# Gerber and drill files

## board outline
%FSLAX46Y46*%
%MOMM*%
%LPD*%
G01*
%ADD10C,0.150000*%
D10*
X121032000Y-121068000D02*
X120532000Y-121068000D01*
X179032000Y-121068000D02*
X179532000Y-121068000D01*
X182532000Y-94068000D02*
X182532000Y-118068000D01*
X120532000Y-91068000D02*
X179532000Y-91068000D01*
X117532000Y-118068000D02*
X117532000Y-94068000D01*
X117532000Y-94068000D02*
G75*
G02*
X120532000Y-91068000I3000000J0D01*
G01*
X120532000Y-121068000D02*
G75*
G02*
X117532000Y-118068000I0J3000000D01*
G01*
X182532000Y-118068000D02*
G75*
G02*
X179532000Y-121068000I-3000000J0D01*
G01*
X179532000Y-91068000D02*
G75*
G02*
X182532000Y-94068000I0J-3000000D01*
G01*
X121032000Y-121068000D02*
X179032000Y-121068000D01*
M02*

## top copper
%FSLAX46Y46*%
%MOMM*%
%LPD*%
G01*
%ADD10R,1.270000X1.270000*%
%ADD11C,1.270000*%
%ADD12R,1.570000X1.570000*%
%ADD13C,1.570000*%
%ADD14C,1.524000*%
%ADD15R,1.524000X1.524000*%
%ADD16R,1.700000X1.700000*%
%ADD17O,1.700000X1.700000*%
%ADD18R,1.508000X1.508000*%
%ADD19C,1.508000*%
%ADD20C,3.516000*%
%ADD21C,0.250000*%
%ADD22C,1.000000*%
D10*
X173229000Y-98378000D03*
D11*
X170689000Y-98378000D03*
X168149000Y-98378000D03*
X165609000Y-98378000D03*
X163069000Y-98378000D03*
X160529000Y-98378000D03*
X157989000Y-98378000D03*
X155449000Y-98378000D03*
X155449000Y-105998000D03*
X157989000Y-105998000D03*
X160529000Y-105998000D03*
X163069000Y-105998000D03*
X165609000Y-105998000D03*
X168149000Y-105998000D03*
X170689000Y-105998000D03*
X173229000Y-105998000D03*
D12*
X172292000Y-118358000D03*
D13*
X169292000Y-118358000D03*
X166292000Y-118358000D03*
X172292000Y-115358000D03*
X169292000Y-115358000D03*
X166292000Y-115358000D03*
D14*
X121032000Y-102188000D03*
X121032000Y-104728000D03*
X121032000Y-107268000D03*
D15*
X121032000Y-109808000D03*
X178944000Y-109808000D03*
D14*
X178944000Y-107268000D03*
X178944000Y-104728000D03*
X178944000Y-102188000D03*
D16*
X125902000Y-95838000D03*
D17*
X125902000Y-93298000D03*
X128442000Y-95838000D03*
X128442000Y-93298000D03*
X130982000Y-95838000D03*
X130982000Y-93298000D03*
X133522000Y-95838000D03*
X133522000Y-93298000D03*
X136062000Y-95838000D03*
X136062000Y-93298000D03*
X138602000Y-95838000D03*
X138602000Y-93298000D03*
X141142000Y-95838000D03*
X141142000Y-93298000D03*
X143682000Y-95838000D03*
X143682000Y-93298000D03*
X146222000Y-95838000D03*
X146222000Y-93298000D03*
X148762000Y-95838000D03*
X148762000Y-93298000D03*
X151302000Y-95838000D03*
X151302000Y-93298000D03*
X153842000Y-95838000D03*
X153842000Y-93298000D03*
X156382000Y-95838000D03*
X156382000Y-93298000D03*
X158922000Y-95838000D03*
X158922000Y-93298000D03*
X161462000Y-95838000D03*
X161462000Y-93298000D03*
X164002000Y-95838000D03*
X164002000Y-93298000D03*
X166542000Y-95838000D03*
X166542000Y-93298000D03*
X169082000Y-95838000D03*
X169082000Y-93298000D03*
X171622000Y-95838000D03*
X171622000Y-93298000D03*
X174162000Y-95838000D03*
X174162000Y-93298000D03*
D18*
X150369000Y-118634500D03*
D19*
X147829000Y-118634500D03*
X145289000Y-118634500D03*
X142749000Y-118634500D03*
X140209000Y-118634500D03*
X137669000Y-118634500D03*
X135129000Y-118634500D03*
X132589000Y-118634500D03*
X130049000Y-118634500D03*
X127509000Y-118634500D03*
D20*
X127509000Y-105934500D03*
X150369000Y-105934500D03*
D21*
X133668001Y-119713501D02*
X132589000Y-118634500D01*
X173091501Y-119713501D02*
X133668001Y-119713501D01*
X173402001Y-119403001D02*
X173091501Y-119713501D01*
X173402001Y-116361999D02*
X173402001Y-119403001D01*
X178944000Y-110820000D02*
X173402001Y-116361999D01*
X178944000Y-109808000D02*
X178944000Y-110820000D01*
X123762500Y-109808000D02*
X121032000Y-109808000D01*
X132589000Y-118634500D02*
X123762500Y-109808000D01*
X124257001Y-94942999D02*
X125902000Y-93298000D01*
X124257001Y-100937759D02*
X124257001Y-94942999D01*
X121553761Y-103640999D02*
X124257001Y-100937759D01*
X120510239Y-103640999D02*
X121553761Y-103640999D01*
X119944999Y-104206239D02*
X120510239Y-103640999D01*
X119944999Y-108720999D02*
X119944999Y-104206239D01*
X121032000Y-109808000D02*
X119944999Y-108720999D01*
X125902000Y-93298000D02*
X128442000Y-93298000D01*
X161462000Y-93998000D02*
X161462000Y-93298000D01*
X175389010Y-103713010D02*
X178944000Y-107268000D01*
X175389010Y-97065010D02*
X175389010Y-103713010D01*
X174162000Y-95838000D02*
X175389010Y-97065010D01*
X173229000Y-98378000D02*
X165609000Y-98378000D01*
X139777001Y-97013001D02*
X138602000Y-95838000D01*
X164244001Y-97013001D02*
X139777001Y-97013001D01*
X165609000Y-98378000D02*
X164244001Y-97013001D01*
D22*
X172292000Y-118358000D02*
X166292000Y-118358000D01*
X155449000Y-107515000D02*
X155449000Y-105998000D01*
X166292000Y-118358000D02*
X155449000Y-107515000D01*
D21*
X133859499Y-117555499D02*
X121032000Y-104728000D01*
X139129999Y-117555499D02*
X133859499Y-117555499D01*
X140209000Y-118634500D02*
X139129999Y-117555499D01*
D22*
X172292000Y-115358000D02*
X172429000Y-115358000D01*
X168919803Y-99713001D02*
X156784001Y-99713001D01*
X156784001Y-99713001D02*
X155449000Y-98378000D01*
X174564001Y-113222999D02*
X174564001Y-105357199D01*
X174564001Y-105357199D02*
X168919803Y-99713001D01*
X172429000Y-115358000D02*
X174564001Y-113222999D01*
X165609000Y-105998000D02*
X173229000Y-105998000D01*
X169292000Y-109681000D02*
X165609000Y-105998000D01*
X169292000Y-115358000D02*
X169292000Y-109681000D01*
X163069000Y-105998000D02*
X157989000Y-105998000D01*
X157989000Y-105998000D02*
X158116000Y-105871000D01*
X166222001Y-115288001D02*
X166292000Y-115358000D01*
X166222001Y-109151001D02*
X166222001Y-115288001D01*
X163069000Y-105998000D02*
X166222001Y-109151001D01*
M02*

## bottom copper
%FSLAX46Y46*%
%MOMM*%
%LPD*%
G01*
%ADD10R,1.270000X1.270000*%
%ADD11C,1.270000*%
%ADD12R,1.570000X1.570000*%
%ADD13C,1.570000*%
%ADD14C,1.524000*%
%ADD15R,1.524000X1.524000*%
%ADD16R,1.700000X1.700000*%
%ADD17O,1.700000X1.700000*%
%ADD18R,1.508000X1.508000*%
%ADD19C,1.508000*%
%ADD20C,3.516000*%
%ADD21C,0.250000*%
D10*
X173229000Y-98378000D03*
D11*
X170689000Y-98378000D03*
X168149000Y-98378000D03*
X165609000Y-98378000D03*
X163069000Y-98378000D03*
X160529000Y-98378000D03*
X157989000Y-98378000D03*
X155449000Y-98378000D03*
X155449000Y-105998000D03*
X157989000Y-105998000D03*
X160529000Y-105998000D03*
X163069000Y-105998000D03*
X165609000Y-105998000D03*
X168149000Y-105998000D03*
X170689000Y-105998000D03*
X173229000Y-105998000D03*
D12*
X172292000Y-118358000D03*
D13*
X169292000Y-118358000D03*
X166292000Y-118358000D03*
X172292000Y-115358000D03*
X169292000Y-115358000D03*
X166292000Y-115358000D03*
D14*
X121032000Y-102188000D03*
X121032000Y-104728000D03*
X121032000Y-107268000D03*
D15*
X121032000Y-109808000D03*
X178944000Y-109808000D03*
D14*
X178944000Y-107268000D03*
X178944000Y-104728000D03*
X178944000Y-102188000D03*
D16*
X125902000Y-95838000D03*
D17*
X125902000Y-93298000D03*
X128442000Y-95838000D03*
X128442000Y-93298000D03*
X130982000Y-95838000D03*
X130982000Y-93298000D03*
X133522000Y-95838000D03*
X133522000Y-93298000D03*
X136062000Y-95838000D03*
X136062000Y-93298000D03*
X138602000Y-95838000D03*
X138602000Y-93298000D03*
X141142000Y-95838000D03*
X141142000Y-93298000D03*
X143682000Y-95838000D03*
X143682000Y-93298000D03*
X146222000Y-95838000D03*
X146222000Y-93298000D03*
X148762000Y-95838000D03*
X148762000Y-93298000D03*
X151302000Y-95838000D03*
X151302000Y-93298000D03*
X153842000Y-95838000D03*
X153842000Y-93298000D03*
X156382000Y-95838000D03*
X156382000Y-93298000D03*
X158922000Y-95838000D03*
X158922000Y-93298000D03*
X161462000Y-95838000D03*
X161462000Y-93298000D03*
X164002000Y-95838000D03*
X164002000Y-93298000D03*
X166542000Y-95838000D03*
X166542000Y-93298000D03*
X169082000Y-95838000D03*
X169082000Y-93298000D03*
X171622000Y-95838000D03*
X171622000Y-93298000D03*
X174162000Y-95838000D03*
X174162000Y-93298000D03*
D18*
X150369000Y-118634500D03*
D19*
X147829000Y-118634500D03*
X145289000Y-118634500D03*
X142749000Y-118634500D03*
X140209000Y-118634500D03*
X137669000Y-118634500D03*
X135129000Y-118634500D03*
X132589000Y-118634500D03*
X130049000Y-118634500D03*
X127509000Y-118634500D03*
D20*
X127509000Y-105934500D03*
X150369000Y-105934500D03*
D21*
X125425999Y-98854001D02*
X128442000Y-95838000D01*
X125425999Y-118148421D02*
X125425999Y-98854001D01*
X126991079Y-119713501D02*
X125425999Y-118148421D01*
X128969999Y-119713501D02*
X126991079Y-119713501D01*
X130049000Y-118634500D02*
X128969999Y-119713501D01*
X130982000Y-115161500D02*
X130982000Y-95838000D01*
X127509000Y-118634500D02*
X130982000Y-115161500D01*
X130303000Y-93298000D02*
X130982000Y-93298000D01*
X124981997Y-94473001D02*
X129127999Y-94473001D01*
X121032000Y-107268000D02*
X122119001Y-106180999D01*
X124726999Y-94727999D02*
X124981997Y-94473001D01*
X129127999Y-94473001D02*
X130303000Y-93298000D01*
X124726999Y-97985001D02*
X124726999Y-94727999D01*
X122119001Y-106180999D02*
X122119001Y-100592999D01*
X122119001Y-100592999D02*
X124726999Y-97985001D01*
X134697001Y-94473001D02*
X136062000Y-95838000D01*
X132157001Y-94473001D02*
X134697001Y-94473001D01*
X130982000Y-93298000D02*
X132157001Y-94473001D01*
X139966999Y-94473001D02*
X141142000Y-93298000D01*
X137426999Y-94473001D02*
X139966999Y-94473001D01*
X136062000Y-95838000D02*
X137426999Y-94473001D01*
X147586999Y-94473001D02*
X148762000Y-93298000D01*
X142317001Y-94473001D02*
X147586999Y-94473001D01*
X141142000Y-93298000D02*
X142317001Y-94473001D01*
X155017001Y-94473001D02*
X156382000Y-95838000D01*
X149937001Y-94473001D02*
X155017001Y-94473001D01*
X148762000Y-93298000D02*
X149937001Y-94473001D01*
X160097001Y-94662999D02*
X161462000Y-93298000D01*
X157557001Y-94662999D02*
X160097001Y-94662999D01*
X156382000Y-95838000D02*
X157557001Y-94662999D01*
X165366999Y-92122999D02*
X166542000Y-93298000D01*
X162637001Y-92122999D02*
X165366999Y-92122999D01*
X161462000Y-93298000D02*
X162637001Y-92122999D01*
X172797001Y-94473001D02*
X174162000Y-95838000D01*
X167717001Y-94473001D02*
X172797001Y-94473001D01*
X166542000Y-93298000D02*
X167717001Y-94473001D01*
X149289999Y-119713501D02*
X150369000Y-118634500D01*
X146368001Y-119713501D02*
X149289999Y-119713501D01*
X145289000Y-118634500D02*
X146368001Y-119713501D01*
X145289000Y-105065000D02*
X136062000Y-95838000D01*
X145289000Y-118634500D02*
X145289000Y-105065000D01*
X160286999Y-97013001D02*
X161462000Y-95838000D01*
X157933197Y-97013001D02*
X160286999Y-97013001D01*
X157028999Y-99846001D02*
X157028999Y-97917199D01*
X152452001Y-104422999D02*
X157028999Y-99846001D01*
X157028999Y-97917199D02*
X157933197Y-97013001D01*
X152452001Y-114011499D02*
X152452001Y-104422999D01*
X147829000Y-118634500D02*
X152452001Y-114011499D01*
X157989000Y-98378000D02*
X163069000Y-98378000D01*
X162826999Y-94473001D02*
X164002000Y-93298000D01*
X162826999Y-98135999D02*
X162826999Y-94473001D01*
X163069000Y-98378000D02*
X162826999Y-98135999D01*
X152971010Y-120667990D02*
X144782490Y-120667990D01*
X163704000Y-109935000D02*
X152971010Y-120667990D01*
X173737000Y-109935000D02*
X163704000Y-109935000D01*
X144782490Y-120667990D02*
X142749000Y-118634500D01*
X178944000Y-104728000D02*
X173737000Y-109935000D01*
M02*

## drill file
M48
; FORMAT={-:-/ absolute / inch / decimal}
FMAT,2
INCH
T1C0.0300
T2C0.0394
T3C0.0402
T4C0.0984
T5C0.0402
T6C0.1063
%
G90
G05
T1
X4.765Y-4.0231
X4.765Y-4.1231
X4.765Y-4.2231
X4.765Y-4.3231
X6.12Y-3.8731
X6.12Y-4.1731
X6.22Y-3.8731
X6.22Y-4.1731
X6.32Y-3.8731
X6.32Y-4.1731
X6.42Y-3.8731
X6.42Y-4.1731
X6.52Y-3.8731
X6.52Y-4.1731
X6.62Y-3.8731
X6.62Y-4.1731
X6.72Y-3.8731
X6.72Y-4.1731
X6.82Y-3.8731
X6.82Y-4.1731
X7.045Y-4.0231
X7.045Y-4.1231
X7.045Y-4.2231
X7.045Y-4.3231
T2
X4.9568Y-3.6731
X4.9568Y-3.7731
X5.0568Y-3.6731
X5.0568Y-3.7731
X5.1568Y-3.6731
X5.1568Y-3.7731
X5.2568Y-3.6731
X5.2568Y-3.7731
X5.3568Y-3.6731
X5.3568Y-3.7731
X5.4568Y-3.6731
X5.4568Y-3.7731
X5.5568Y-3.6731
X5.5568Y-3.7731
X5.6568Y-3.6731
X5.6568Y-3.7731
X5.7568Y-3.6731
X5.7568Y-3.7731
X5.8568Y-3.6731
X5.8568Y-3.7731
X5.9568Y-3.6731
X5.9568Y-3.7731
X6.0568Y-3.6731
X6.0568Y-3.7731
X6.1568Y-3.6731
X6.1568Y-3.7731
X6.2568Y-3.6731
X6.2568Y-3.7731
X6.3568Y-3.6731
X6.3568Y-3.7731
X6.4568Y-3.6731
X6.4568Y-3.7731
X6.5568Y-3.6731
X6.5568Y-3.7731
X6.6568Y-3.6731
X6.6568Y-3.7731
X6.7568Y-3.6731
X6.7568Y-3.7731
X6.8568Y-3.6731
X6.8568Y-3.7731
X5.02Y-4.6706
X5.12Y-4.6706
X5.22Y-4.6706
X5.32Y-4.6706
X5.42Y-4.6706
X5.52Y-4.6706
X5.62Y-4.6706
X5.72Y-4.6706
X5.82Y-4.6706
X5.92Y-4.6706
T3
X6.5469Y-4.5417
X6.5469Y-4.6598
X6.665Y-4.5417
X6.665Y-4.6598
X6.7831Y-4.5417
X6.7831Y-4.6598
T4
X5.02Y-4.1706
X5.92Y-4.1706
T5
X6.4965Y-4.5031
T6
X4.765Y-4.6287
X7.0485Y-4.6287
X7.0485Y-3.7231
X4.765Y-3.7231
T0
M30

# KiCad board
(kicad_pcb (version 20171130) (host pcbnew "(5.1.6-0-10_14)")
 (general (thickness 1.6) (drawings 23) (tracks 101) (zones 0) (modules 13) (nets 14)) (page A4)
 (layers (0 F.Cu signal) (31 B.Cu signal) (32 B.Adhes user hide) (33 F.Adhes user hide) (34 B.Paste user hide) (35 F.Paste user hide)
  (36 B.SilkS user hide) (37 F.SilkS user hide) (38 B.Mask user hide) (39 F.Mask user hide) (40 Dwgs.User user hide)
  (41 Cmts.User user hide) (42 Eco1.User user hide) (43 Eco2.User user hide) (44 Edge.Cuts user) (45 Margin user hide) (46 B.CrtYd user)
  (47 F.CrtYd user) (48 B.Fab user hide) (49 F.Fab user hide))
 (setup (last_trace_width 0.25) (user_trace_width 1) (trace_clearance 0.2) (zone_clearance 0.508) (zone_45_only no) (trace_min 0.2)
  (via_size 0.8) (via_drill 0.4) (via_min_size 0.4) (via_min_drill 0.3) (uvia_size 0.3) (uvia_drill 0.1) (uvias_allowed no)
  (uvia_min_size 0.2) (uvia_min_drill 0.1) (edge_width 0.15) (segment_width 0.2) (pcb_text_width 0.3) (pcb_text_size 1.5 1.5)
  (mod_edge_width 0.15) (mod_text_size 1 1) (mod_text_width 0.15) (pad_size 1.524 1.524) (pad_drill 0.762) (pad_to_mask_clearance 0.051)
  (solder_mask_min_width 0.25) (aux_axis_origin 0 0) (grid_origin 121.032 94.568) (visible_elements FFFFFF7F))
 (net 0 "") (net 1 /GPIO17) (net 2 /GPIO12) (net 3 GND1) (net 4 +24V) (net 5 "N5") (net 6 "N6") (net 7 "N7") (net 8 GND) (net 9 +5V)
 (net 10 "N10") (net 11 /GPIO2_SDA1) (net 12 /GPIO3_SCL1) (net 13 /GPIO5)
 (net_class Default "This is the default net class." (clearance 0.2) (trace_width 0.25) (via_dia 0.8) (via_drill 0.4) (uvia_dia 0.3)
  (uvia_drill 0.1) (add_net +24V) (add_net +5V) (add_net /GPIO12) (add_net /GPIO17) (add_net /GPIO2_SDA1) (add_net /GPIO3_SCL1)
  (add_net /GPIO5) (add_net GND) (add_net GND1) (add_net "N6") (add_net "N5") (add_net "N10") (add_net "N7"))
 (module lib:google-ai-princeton (layer F.Cu) (at 148.972 107.395)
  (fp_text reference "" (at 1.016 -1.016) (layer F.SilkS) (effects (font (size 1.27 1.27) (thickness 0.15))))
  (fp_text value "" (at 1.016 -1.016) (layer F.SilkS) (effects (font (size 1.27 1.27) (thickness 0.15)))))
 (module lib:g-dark (layer F.Cu) (at 158.624 114.38)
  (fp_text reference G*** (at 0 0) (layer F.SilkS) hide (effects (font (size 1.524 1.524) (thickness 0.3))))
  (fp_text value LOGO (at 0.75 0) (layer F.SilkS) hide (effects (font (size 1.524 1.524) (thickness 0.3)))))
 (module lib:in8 (layer F.Cu) (at 148.337 100.156)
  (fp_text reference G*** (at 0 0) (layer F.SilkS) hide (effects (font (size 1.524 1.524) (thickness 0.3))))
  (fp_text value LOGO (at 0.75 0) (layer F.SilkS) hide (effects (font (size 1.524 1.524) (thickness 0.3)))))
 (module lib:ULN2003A (layer F.Cu) (at 173.229 98.378 270)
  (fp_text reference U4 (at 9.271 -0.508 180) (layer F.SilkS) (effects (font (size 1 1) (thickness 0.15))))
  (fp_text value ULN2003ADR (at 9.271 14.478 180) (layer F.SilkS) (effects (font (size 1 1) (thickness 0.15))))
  (pad 1 thru_hole rect (at 0 0 270) (size 1.27 1.27) (drill 0.762) (layers *.Cu *.Mask) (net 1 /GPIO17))
  (pad 2 thru_hole circle (at 0 2.54 270) (size 1.27 1.27) (drill 0.762) (layers *.Cu *.Mask) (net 1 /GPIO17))
  (pad 3 thru_hole circle (at 0 5.08 270) (size 1.27 1.27) (drill 0.762) (layers *.Cu *.Mask) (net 1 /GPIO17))
  (pad 4 thru_hole circle (at 0 7.62 270) (size 1.27 1.27) (drill 0.762) (layers *.Cu *.Mask) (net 1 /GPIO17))
  (pad 5 thru_hole circle (at 0 10.16 270) (size 1.27 1.27) (drill 0.762) (layers *.Cu *.Mask) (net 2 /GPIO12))
  (pad 6 thru_hole circle (at 0 12.7 270) (size 1.27 1.27) (drill 0.762) (layers *.Cu *.Mask) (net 2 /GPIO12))
  (pad 7 thru_hole circle (at 0 15.24 270) (size 1.27 1.27) (drill 0.762) (layers *.Cu *.Mask) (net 2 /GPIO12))
  (pad 8 thru_hole circle (at 0 17.78 270) (size 1.27 1.27) (drill 0.762) (layers *.Cu *.Mask) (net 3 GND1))
  (pad 9 thru_hole circle (at 7.62 17.78 270) (size 1.27 1.27) (drill 0.762) (layers *.Cu *.Mask) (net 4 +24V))
  (pad 10 thru_hole circle (at 7.62 15.24 270) (size 1.27 1.27) (drill 0.762) (layers *.Cu *.Mask) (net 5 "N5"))
  (pad 11 thru_hole circle (at 7.62 12.7 270) (size 1.27 1.27) (drill 0.762) (layers *.Cu *.Mask) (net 5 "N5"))
  (pad 12 thru_hole circle (at 7.62 10.16 270) (size 1.27 1.27) (drill 0.762) (layers *.Cu *.Mask) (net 5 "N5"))
  (pad 13 thru_hole circle (at 7.62 7.62 270) (size 1.27 1.27) (drill 0.762) (layers *.Cu *.Mask) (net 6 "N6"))
  (pad 14 thru_hole circle (at 7.62 5.08 270) (size 1.27 1.27) (drill 0.762) (layers *.Cu *.Mask) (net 6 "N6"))
  (pad 15 thru_hole circle (at 7.62 2.54 270) (size 1.27 1.27) (drill 0.762) (layers *.Cu *.Mask) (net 6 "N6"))
  (pad 16 thru_hole circle (at 7.62 0 270) (size 1.27 1.27) (drill 0.762) (layers *.Cu *.Mask) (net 6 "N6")))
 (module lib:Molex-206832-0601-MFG (layer F.Cu) (at 169.292 116.158)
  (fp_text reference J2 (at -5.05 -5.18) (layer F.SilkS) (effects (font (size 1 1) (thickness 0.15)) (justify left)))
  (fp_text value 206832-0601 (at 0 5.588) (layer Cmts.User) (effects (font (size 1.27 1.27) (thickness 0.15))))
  (pad 1 thru_hole rect (at 3 2.2 90) (size 1.57 1.57) (drill 1.02) (layers *.Cu) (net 4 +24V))
  (pad 3 thru_hole circle (at 0 2.2) (size 1.57 1.57) (drill 1.02) (layers *.Cu) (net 4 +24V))
  (pad 5 thru_hole circle (at -3 2.2) (size 1.57 1.57) (drill 1.02) (layers *.Cu) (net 4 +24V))
  (pad 2 thru_hole circle (at 3 -0.8) (size 1.57 1.57) (drill 1.02) (layers *.Cu) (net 3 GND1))
  (pad 4 thru_hole circle (at 0 -0.8) (size 1.57 1.57) (drill 1.02) (layers *.Cu) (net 6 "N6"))
  (pad 6 thru_hole circle (at -3 -0.8) (size 1.57 1.57) (drill 1.02) (layers *.Cu) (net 5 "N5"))
  (pad ~ np_thru_hole circle (at -4.28 -1.78) (size 1.02 1.02) (drill 1.02) (layers *.Cu *.Mask)))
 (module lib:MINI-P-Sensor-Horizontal (layer F.Cu) (at 121.032 109.808 90)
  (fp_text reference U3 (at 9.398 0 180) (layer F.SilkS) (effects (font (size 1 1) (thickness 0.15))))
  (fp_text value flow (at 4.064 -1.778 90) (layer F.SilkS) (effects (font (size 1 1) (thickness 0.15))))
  (pad 4 thru_hole circle (at 7.62 0 90) (size 1.524 1.524) (drill 0.762) (layers *.Cu *.Mask))
  (pad 3 thru_hole circle (at 5.08 0 90) (size 1.524 1.524) (drill 0.762) (layers *.Cu *.Mask) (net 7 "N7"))
  (pad 2 thru_hole circle (at 2.54 0 90) (size 1.524 1.524) (drill 0.762) (layers *.Cu *.Mask) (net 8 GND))
  (pad 1 thru_hole rect (at 0 0 90) (size 1.524 1.524) (drill 0.762) (layers *.Cu *.Mask) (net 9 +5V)))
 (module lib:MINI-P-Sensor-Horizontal (layer F.Cu) (at 178.944 109.808 90)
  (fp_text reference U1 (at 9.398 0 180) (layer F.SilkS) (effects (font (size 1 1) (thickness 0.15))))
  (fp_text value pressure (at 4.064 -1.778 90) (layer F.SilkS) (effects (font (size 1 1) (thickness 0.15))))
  (pad 1 thru_hole rect (at 0 0 90) (size 1.524 1.524) (drill 0.762) (layers *.Cu *.Mask) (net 9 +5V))
  (pad 2 thru_hole circle (at 2.54 0 90) (size 1.524 1.524) (drill 0.762) (layers *.Cu *.Mask) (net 8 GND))
  (pad 3 thru_hole circle (at 5.08 0 90) (size 1.524 1.524) (drill 0.762) (layers *.Cu *.Mask) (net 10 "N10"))
  (pad 4 thru_hole circle (at 7.62 0 90) (size 1.524 1.524) (drill 0.762) (layers *.Cu *.Mask)))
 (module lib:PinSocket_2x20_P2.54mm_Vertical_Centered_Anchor (layer B.Cu) (at 125.902 95.838 270)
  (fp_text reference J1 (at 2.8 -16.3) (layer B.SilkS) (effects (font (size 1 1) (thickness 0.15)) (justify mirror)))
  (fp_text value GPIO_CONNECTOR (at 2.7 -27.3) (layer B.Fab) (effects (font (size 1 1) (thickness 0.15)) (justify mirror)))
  (pad 1 thru_hole rect (at 0 0 270) (size 1.7 1.7) (drill 1) (layers *.Cu *.Mask))
  (pad 2 thru_hole oval (at -2.54 0 270) (size 1.7 1.7) (drill 1) (layers *.Cu *.Mask) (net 9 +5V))
  (pad 3 thru_hole oval (at 0 -2.54 270) (size 1.7 1.7) (drill 1) (layers *.Cu *.Mask) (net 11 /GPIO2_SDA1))
  (pad 4 thru_hole oval (at -2.54 -2.54 270) (size 1.7 1.7) (drill 1) (layers *.Cu *.Mask) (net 9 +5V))
  (pad 5 thru_hole oval (at 0 -5.08 270) (size 1.7 1.7) (drill 1) (layers *.Cu *.Mask) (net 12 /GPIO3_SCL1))
  (pad 6 thru_hole oval (at -2.54 -5.08 270) (size 1.7 1.7) (drill 1) (layers *.Cu *.Mask) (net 8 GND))
  (pad 7 thru_hole oval (at 0 -7.62 270) (size 1.7 1.7) (drill 1) (layers *.Cu *.Mask))
  (pad 8 thru_hole oval (at -2.54 -7.62 270) (size 1.7 1.7) (drill 1) (layers *.Cu *.Mask))
  (pad 9 thru_hole oval (at 0 -10.16 270) (size 1.7 1.7) (drill 1) (layers *.Cu *.Mask) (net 8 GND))
  (pad 10 thru_hole oval (at -2.54 -10.16 270) (size 1.7 1.7) (drill 1) (layers *.Cu *.Mask))
  (pad 11 thru_hole oval (at 0 -12.7 270) (size 1.7 1.7) (drill 1) (layers *.Cu *.Mask) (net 1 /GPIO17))
  (pad 12 thru_hole oval (at -2.54 -12.7 270) (size 1.7 1.7) (drill 1) (layers *.Cu *.Mask))
  (pad 13 thru_hole oval (at 0 -15.24 270) (size 1.7 1.7) (drill 1) (layers *.Cu *.Mask))
  (pad 14 thru_hole oval (at -2.54 -15.24 270) (size 1.7 1.7) (drill 1) (layers *.Cu *.Mask) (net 8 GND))
  (pad 15 thru_hole oval (at 0 -17.78 270) (size 1.7 1.7) (drill 1) (layers *.Cu *.Mask))
  (pad 16 thru_hole oval (at -2.54 -17.78 270) (size 1.7 1.7) (drill 1) (layers *.Cu *.Mask))
  (pad 17 thru_hole oval (at 0 -20.32 270) (size 1.7 1.7) (drill 1) (layers *.Cu *.Mask))
  (pad 18 thru_hole oval (at -2.54 -20.32 270) (size 1.7 1.7) (drill 1) (layers *.Cu *.Mask))
  (pad 19 thru_hole oval (at 0 -22.86 270) (size 1.7 1.7) (drill 1) (layers *.Cu *.Mask))
  (pad 20 thru_hole oval (at -2.54 -22.86 270) (size 1.7 1.7) (drill 1) (layers *.Cu *.Mask) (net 8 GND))
  (pad 21 thru_hole oval (at 0 -25.4 270) (size 1.7 1.7) (drill 1) (layers *.Cu *.Mask))
  (pad 22 thru_hole oval (at -2.54 -25.4 270) (size 1.7 1.7) (drill 1) (layers *.Cu *.Mask))
  (pad 23 thru_hole oval (at 0 -27.94 270) (size 1.7 1.7) (drill 1) (layers *.Cu *.Mask))
  (pad 24 thru_hole oval (at -2.54 -27.94 270) (size 1.7 1.7) (drill 1) (layers *.Cu *.Mask))
  (pad 25 thru_hole oval (at 0 -30.48 270) (size 1.7 1.7) (drill 1) (layers *.Cu *.Mask) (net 8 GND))
  (pad 26 thru_hole oval (at -2.54 -30.48 270) (size 1.7 1.7) (drill 1) (layers *.Cu *.Mask))
  (pad 27 thru_hole oval (at 0 -33.02 270) (size 1.7 1.7) (drill 1) (layers *.Cu *.Mask))
  (pad 28 thru_hole oval (at -2.54 -33.02 270) (size 1.7 1.7) (drill 1) (layers *.Cu *.Mask))
  (pad 29 thru_hole oval (at 0 -35.56 270) (size 1.7 1.7) (drill 1) (layers *.Cu *.Mask) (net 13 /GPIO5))
  (pad 30 thru_hole oval (at -2.54 -35.56 270) (size 1.7 1.7) (drill 1) (layers *.Cu *.Mask) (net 8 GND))
  (pad 31 thru_hole oval (at 0 -38.1 270) (size 1.7 1.7) (drill 1) (layers *.Cu *.Mask))
  (pad 32 thru_hole oval (at -2.54 -38.1 270) (size 1.7 1.7) (drill 1) (layers *.Cu *.Mask) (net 2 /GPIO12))
  (pad 33 thru_hole oval (at 0 -40.64 270) (size 1.7 1.7) (drill 1) (layers *.Cu *.Mask))
  (pad 34 thru_hole oval (at -2.54 -40.64 270) (size 1.7 1.7) (drill 1) (layers *.Cu *.Mask) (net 8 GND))
  (pad 35 thru_hole oval (at 0 -43.18 270) (size 1.7 1.7) (drill 1) (layers *.Cu *.Mask))
  (pad 36 thru_hole oval (at -2.54 -43.18 270) (size 1.7 1.7) (drill 1) (layers *.Cu *.Mask))
  (pad 37 thru_hole oval (at 0 -45.72 270) (size 1.7 1.7) (drill 1) (layers *.Cu *.Mask))
  (pad 38 thru_hole oval (at -2.54 -45.72 270) (size 1.7 1.7) (drill 1) (layers *.Cu *.Mask))
  (pad 39 thru_hole oval (at 0 -48.26 270) (size 1.7 1.7) (drill 1) (layers *.Cu *.Mask) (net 8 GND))
  (pad 40 thru_hole oval (at -2.54 -48.26 270) (size 1.7 1.7) (drill 1) (layers *.Cu *.Mask)))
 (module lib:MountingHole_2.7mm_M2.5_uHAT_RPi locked (layer F.Cu) (at 121.032 94.568)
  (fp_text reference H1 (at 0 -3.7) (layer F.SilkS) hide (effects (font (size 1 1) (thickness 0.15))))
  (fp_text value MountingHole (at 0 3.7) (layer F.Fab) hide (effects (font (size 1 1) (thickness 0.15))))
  (pad "" np_thru_hole circle (at 0 0) (size 2.7 2.7) (drill 2.7) (layers *.Cu *.Mask) (clearance 1.75)))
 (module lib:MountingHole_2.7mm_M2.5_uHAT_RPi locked (layer F.Cu) (at 179.032 94.568)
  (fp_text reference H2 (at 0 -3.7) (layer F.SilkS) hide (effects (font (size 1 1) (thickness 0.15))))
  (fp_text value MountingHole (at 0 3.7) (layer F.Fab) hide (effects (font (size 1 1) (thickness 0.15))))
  (pad "" np_thru_hole circle (at 0 0) (size 2.7 2.7) (drill 2.7) (layers *.Cu *.Mask) (clearance 1.75)))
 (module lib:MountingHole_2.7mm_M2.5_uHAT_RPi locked (layer F.Cu) (at 179.032 117.568)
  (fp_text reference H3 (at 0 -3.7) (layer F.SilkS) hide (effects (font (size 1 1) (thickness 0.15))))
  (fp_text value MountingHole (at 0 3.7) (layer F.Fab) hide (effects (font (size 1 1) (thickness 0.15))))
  (pad "" np_thru_hole circle (at 0 0) (size 2.7 2.7) (drill 2.7) (layers *.Cu *.Mask) (clearance 1.75)))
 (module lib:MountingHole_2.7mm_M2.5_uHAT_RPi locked (layer F.Cu) (at 121.032 117.568)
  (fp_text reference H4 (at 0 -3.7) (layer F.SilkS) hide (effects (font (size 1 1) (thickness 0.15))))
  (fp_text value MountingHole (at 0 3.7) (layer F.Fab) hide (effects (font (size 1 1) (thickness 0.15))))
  (pad "" np_thru_hole circle (at 0 0) (size 2.7 2.7) (drill 2.7) (layers *.Cu *.Mask) (clearance 1.75)))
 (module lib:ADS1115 (layer F.Cu) (at 138.939 111.967)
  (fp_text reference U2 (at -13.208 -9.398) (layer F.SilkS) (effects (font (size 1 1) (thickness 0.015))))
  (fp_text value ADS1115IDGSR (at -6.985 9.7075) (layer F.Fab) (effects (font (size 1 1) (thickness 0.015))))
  (pad 1 thru_hole rect (at 11.43 6.6675) (size 1.508 1.508) (drill 1) (layers *.Cu *.Mask) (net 8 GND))
  (pad 2 thru_hole circle (at 8.89 6.6675) (size 1.508 1.508) (drill 1) (layers *.Cu *.Mask) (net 13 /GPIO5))
  (pad 3 thru_hole circle (at 6.35 6.6675) (size 1.508 1.508) (drill 1) (layers *.Cu *.Mask) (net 8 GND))
  (pad 4 thru_hole circle (at 3.81 6.6675) (size 1.508 1.508) (drill 1) (layers *.Cu *.Mask) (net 10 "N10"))
  (pad 5 thru_hole circle (at 1.27 6.6675) (size 1.508 1.508) (drill 1) (layers *.Cu *.Mask) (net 7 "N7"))
  (pad 6 thru_hole circle (at -1.27 6.6675) (size 1.508 1.508) (drill 1) (layers *.Cu *.Mask))
  (pad 7 thru_hole circle (at -3.81 6.6675) (size 1.508 1.508) (drill 1) (layers *.Cu *.Mask))
  (pad 8 thru_hole circle (at -6.35 6.6675) (size 1.508 1.508) (drill 1) (layers *.Cu *.Mask) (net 9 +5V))
  (pad 9 thru_hole circle (at -8.89 6.6675) (size 1.508 1.508) (drill 1) (layers *.Cu *.Mask) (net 11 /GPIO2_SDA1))
  (pad 10 thru_hole circle (at -11.43 6.6675) (size 1.508 1.508) (drill 1) (layers *.Cu *.Mask) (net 12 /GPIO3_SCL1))
  (pad P1 thru_hole circle (at -11.43 -6.0325) (size 3.516 3.516) (drill 2.5) (layers *.Cu *.Mask))
  (pad P2 thru_hole circle (at 11.43 -6.0325) (size 3.516 3.516) (drill 2.5) (layers *.Cu *.Mask)))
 (gr_line (start 121.032 121.068) (end 120.532 121.068) (layer Edge.Cuts) (width 0.15))
 (gr_line (start 179.032 121.068) (end 179.532 121.068) (layer Edge.Cuts) (width 0.15))
 (gr_line (start 182.532 94.068) (end 182.532 118.068) (layer Edge.Cuts) (width 0.15))
 (gr_line (start 120.532 91.068) (end 179.532 91.068) (layer Edge.Cuts) (width 0.15))
 (gr_line (start 117.532 118.068) (end 117.532 94.068) (layer Edge.Cuts) (width 0.15))
 (gr_arc (start 120.532 94.068) (end 120.532 91.068) (angle -90) (layer Edge.Cuts) (width 0.15))
 (gr_arc (start 120.532 118.068) (end 117.532 118.068) (angle -90) (layer Edge.Cuts) (width 0.15))
 (gr_arc (start 179.532 118.068) (end 179.532 121.068) (angle -90) (layer Edge.Cuts) (width 0.15))
 (gr_arc (start 179.532 94.068) (end 182.532 94.068) (angle -90) (layer Edge.Cuts) (width 0.15))
 (gr_line (start 121.032 121.068) (end 179.032 121.068) (layer Edge.Cuts) (width 0.15))
 (segment (start 133.668001 119.713501) (end 132.589 118.6345) (width 0.25) (layer F.Cu) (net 9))
 (segment (start 173.091501 119.713501) (end 133.668001 119.713501) (width 0.25) (layer F.Cu) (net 9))
 (segment (start 173.402001 119.403001) (end 173.091501 119.713501) (width 0.25) (layer F.Cu) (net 9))
 (segment (start 173.402001 116.361999) (end 173.402001 119.403001) (width 0.25) (layer F.Cu) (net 9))
 (segment (start 178.944 110.82) (end 173.402001 116.361999) (width 0.25) (layer F.Cu) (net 9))
 (segment (start 178.944 109.808) (end 178.944 110.82) (width 0.25) (layer F.Cu) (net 9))
 (segment (start 123.7625 109.808) (end 121.032 109.808) (width 0.25) (layer F.Cu) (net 9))
 (segment (start 132.589 118.6345) (end 123.7625 109.808) (width 0.25) (layer F.Cu) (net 9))
 (segment (start 124.257001 94.942999) (end 125.902 93.298) (width 0.25) (layer F.Cu) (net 9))
 (segment (start 124.257001 100.937759) (end 124.257001 94.942999) (width 0.25) (layer F.Cu) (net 9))
 (segment (start 121.553761 103.640999) (end 124.257001 100.937759) (width 0.25) (layer F.Cu) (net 9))
 (segment (start 120.510239 103.640999) (end 121.553761 103.640999) (width 0.25) (layer F.Cu) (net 9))
 (segment (start 119.944999 104.206239) (end 120.510239 103.640999) (width 0.25) (layer F.Cu) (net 9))
 (segment (start 119.944999 108.720999) (end 119.944999 104.206239) (width 0.25) (layer F.Cu) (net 9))
 (segment (start 121.032 109.808) (end 119.944999 108.720999) (width 0.25) (layer F.Cu) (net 9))
 (segment (start 125.902 93.298) (end 128.442 93.298) (width 0.25) (layer F.Cu) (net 9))
 (segment (start 125.425999 98.854001) (end 128.442 95.838) (width 0.25) (layer B.Cu) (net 11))
 (segment (start 125.425999 118.148421) (end 125.425999 98.854001) (width 0.25) (layer B.Cu) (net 11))
 (segment (start 126.991079 119.713501) (end 125.425999 118.148421) (width 0.25) (layer B.Cu) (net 11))
 (segment (start 128.969999 119.713501) (end 126.991079 119.713501) (width 0.25) (layer B.Cu) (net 11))
 (segment (start 130.049 118.6345) (end 128.969999 119.713501) (width 0.25) (layer B.Cu) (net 11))
 (segment (start 130.982 115.1615) (end 130.982 95.838) (width 0.25) (layer B.Cu) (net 12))
 (segment (start 127.509 118.6345) (end 130.982 115.1615) (width 0.25) (layer B.Cu) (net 12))
 (segment (start 161.462 93.998) (end 161.462 93.298) (width 0.25) (layer F.Cu) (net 8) (status 30))
 (segment (start 130.303 93.298) (end 130.982 93.298) (width 0.25) (layer B.Cu) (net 8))
 (segment (start 124.981997 94.473001) (end 129.127999 94.473001) (width 0.25) (layer B.Cu) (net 8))
 (segment (start 121.032 107.268) (end 122.119001 106.180999) (width 0.25) (layer B.Cu) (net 8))
 (segment (start 124.726999 94.727999) (end 124.981997 94.473001) (width 0.25) (layer B.Cu) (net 8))
 (segment (start 129.127999 94.473001) (end 130.303 93.298) (width 0.25) (layer B.Cu) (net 8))
 (segment (start 124.726999 97.985001) (end 124.726999 94.727999) (width 0.25) (layer B.Cu) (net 8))
 (segment (start 122.119001 106.180999) (end 122.119001 100.592999) (width 0.25) (layer B.Cu) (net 8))
 (segment (start 122.119001 100.592999) (end 124.726999 97.985001) (width 0.25) (layer B.Cu) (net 8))
 (segment (start 134.697001 94.473001) (end 136.062 95.838) (width 0.25) (layer B.Cu) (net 8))
 (segment (start 132.157001 94.473001) (end 134.697001 94.473001) (width 0.25) (layer B.Cu) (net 8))
 (segment (start 130.982 93.298) (end 132.157001 94.473001) (width 0.25) (layer B.Cu) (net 8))
 (segment (start 139.966999 94.473001) (end 141.142 93.298) (width 0.25) (layer B.Cu) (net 8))
 (segment (start 137.426999 94.473001) (end 139.966999 94.473001) (width 0.25) (layer B.Cu) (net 8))
 (segment (start 136.062 95.838) (end 137.426999 94.473001) (width 0.25) (layer B.Cu) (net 8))
 (segment (start 147.586999 94.473001) (end 148.762 93.298) (width 0.25) (layer B.Cu) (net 8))
 (segment (start 142.317001 94.473001) (end 147.586999 94.473001) (width 0.25) (layer B.Cu) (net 8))
 (segment (start 141.142 93.298) (end 142.317001 94.473001) (width 0.25) (layer B.Cu) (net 8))
 (segment (start 155.017001 94.473001) (end 156.382 95.838) (width 0.25) (layer B.Cu) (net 8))
 (segment (start 149.937001 94.473001) (end 155.017001 94.473001) (width 0.25) (layer B.Cu) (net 8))
 (segment (start 148.762 93.298) (end 149.937001 94.473001) (width 0.25) (layer B.Cu) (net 8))
 (segment (start 160.097001 94.662999) (end 161.462 93.298) (width 0.25) (layer B.Cu) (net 8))
 (segment (start 157.557001 94.662999) (end 160.097001 94.662999) (width 0.25) (layer B.Cu) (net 8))
 (segment (start 156.382 95.838) (end 157.557001 94.662999) (width 0.25) (layer B.Cu) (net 8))
 (segment (start 165.366999 92.122999) (end 166.542 93.298) (width 0.25) (layer B.Cu) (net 8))
 (segment (start 162.637001 92.122999) (end 165.366999 92.122999) (width 0.25) (layer B.Cu) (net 8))
 (segment (start 161.462 93.298) (end 162.637001 92.122999) (width 0.25) (layer B.Cu) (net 8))
 (segment (start 172.797001 94.473001) (end 174.162 95.838) (width 0.25) (layer B.Cu) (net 8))
 (segment (start 167.717001 94.473001) (end 172.797001 94.473001) (width 0.25) (layer B.Cu) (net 8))
 (segment (start 166.542 93.298) (end 167.717001 94.473001) (width 0.25) (layer B.Cu) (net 8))
 (segment (start 175.38901 103.71301) (end 178.944 107.268) (width 0.25) (layer F.Cu) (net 8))
 (segment (start 175.38901 97.06501) (end 175.38901 103.71301) (width 0.25) (layer F.Cu) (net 8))
 (segment (start 174.162 95.838) (end 175.38901 97.06501) (width 0.25) (layer F.Cu) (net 8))
 (segment (start 149.289999 119.713501) (end 150.369 118.6345) (width 0.25) (layer B.Cu) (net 8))
 (segment (start 146.368001 119.713501) (end 149.289999 119.713501) (width 0.25) (layer B.Cu) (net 8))
 (segment (start 145.289 118.6345) (end 146.368001 119.713501) (width 0.25) (layer B.Cu) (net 8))
 (segment (start 145.289 105.065) (end 136.062 95.838) (width 0.25) (layer B.Cu) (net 8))
 (segment (start 145.289 118.6345) (end 145.289 105.065) (width 0.25) (layer B.Cu) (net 8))
 (segment (start 160.286999 97.013001) (end 161.462 95.838) (width 0.25) (layer B.Cu) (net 13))
 (segment (start 157.933197 97.013001) (end 160.286999 97.013001) (width 0.25) (layer B.Cu) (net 13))
 (segment (start 157.028999 99.846001) (end 157.028999 97.917199) (width 0.25) (layer B.Cu) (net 13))
 (segment (start 152.452001 104.422999) (end 157.028999 99.846001) (width 0.25) (layer B.Cu) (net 13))
 (segment (start 157.028999 97.917199) (end 157.933197 97.013001) (width 0.25) (layer B.Cu) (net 13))
 (segment (start 152.452001 114.011499) (end 152.452001 104.422999) (width 0.25) (layer B.Cu) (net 13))
 (segment (start 147.829 118.6345) (end 152.452001 114.011499) (width 0.25) (layer B.Cu) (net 13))
 (segment (start 157.989 98.378) (end 163.069 98.378) (width 0.25) (layer B.Cu) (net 2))
 (segment (start 162.826999 94.473001) (end 164.002 93.298) (width 0.25) (layer B.Cu) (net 2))
 (segment (start 162.826999 98.135999) (end 162.826999 94.473001) (width 0.25) (layer B.Cu) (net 2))
 (segment (start 163.069 98.378) (end 162.826999 98.135999) (width 0.25) (layer B.Cu) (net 2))
 (segment (start 173.229 98.378) (end 165.609 98.378) (width 0.25) (layer F.Cu) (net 1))
 (segment (start 139.777001 97.013001) (end 138.602 95.838) (width 0.25) (layer F.Cu) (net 1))
 (segment (start 164.244001 97.013001) (end 139.777001 97.013001) (width 0.25) (layer F.Cu) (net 1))
 (segment (start 165.609 98.378) (end 164.244001 97.013001) (width 0.25) (layer F.Cu) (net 1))
 (segment (start 172.292 118.358) (end 166.292 118.358) (width 1) (layer F.Cu) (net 4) (status 30))
 (segment (start 155.449 107.515) (end 155.449 105.998) (width 1) (layer F.Cu) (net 4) (status 20))
 (segment (start 166.292 118.358) (end 155.449 107.515) (width 1) (layer F.Cu) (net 4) (status 10))
 (segment (start 152.97101 120.66799) (end 144.78249 120.66799) (width 0.25) (layer B.Cu) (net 10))
 (segment (start 163.704 109.935) (end 152.97101 120.66799) (width 0.25) (layer B.Cu) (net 10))
 (segment (start 173.737 109.935) (end 163.704 109.935) (width 0.25) (layer B.Cu) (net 10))
 (segment (start 144.78249 120.66799) (end 142.749 118.6345) (width 0.25) (layer B.Cu) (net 10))
 (segment (start 178.944 104.728) (end 173.737 109.935) (width 0.25) (layer B.Cu) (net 10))
 (segment (start 133.859499 117.555499) (end 121.032 104.728) (width 0.25) (layer F.Cu) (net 7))
 (segment (start 139.129999 117.555499) (end 133.859499 117.555499) (width 0.25) (layer F.Cu) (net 7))
 (segment (start 140.209 118.6345) (end 139.129999 117.555499) (width 0.25) (layer F.Cu) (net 7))
 (segment (start 172.292 115.358) (end 172.429 115.358) (width 1) (layer F.Cu) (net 3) (status 30))
 (segment (start 168.919803 99.713001) (end 156.784001 99.713001) (width 1) (layer F.Cu) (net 3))
 (segment (start 156.784001 99.713001) (end 155.449 98.378) (width 1) (layer F.Cu) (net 3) (status 20))
 (segment (start 174.564001 113.222999) (end 174.564001 105.357199) (width 1) (layer F.Cu) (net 3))
 (segment (start 174.564001 105.357199) (end 168.919803 99.713001) (width 1) (layer F.Cu) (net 3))
 (segment (start 172.429 115.358) (end 174.564001 113.222999) (width 1) (layer F.Cu) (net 3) (status 10))
 (segment (start 165.609 105.998) (end 173.229 105.998) (width 1) (layer F.Cu) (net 6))
 (segment (start 169.292 109.681) (end 165.609 105.998) (width 1) (layer F.Cu) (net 6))
 (segment (start 169.292 115.358) (end 169.292 109.681) (width 1) (layer F.Cu) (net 6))
 (segment (start 163.069 105.998) (end 157.989 105.998) (width 1) (layer F.Cu) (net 5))
 (segment (start 157.989 105.998) (end 158.116 105.871) (width 1) (layer F.Cu) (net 5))
 (segment (start 166.222001 115.288001) (end 166.292 115.358) (width 1) (layer F.Cu) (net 5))
 (segment (start 166.222001 109.151001) (end 166.222001 115.288001) (width 1) (layer F.Cu) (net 5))
 (segment (start 163.069 105.998) (end 166.222001 109.151001) (width 1) (layer F.Cu) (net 5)))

